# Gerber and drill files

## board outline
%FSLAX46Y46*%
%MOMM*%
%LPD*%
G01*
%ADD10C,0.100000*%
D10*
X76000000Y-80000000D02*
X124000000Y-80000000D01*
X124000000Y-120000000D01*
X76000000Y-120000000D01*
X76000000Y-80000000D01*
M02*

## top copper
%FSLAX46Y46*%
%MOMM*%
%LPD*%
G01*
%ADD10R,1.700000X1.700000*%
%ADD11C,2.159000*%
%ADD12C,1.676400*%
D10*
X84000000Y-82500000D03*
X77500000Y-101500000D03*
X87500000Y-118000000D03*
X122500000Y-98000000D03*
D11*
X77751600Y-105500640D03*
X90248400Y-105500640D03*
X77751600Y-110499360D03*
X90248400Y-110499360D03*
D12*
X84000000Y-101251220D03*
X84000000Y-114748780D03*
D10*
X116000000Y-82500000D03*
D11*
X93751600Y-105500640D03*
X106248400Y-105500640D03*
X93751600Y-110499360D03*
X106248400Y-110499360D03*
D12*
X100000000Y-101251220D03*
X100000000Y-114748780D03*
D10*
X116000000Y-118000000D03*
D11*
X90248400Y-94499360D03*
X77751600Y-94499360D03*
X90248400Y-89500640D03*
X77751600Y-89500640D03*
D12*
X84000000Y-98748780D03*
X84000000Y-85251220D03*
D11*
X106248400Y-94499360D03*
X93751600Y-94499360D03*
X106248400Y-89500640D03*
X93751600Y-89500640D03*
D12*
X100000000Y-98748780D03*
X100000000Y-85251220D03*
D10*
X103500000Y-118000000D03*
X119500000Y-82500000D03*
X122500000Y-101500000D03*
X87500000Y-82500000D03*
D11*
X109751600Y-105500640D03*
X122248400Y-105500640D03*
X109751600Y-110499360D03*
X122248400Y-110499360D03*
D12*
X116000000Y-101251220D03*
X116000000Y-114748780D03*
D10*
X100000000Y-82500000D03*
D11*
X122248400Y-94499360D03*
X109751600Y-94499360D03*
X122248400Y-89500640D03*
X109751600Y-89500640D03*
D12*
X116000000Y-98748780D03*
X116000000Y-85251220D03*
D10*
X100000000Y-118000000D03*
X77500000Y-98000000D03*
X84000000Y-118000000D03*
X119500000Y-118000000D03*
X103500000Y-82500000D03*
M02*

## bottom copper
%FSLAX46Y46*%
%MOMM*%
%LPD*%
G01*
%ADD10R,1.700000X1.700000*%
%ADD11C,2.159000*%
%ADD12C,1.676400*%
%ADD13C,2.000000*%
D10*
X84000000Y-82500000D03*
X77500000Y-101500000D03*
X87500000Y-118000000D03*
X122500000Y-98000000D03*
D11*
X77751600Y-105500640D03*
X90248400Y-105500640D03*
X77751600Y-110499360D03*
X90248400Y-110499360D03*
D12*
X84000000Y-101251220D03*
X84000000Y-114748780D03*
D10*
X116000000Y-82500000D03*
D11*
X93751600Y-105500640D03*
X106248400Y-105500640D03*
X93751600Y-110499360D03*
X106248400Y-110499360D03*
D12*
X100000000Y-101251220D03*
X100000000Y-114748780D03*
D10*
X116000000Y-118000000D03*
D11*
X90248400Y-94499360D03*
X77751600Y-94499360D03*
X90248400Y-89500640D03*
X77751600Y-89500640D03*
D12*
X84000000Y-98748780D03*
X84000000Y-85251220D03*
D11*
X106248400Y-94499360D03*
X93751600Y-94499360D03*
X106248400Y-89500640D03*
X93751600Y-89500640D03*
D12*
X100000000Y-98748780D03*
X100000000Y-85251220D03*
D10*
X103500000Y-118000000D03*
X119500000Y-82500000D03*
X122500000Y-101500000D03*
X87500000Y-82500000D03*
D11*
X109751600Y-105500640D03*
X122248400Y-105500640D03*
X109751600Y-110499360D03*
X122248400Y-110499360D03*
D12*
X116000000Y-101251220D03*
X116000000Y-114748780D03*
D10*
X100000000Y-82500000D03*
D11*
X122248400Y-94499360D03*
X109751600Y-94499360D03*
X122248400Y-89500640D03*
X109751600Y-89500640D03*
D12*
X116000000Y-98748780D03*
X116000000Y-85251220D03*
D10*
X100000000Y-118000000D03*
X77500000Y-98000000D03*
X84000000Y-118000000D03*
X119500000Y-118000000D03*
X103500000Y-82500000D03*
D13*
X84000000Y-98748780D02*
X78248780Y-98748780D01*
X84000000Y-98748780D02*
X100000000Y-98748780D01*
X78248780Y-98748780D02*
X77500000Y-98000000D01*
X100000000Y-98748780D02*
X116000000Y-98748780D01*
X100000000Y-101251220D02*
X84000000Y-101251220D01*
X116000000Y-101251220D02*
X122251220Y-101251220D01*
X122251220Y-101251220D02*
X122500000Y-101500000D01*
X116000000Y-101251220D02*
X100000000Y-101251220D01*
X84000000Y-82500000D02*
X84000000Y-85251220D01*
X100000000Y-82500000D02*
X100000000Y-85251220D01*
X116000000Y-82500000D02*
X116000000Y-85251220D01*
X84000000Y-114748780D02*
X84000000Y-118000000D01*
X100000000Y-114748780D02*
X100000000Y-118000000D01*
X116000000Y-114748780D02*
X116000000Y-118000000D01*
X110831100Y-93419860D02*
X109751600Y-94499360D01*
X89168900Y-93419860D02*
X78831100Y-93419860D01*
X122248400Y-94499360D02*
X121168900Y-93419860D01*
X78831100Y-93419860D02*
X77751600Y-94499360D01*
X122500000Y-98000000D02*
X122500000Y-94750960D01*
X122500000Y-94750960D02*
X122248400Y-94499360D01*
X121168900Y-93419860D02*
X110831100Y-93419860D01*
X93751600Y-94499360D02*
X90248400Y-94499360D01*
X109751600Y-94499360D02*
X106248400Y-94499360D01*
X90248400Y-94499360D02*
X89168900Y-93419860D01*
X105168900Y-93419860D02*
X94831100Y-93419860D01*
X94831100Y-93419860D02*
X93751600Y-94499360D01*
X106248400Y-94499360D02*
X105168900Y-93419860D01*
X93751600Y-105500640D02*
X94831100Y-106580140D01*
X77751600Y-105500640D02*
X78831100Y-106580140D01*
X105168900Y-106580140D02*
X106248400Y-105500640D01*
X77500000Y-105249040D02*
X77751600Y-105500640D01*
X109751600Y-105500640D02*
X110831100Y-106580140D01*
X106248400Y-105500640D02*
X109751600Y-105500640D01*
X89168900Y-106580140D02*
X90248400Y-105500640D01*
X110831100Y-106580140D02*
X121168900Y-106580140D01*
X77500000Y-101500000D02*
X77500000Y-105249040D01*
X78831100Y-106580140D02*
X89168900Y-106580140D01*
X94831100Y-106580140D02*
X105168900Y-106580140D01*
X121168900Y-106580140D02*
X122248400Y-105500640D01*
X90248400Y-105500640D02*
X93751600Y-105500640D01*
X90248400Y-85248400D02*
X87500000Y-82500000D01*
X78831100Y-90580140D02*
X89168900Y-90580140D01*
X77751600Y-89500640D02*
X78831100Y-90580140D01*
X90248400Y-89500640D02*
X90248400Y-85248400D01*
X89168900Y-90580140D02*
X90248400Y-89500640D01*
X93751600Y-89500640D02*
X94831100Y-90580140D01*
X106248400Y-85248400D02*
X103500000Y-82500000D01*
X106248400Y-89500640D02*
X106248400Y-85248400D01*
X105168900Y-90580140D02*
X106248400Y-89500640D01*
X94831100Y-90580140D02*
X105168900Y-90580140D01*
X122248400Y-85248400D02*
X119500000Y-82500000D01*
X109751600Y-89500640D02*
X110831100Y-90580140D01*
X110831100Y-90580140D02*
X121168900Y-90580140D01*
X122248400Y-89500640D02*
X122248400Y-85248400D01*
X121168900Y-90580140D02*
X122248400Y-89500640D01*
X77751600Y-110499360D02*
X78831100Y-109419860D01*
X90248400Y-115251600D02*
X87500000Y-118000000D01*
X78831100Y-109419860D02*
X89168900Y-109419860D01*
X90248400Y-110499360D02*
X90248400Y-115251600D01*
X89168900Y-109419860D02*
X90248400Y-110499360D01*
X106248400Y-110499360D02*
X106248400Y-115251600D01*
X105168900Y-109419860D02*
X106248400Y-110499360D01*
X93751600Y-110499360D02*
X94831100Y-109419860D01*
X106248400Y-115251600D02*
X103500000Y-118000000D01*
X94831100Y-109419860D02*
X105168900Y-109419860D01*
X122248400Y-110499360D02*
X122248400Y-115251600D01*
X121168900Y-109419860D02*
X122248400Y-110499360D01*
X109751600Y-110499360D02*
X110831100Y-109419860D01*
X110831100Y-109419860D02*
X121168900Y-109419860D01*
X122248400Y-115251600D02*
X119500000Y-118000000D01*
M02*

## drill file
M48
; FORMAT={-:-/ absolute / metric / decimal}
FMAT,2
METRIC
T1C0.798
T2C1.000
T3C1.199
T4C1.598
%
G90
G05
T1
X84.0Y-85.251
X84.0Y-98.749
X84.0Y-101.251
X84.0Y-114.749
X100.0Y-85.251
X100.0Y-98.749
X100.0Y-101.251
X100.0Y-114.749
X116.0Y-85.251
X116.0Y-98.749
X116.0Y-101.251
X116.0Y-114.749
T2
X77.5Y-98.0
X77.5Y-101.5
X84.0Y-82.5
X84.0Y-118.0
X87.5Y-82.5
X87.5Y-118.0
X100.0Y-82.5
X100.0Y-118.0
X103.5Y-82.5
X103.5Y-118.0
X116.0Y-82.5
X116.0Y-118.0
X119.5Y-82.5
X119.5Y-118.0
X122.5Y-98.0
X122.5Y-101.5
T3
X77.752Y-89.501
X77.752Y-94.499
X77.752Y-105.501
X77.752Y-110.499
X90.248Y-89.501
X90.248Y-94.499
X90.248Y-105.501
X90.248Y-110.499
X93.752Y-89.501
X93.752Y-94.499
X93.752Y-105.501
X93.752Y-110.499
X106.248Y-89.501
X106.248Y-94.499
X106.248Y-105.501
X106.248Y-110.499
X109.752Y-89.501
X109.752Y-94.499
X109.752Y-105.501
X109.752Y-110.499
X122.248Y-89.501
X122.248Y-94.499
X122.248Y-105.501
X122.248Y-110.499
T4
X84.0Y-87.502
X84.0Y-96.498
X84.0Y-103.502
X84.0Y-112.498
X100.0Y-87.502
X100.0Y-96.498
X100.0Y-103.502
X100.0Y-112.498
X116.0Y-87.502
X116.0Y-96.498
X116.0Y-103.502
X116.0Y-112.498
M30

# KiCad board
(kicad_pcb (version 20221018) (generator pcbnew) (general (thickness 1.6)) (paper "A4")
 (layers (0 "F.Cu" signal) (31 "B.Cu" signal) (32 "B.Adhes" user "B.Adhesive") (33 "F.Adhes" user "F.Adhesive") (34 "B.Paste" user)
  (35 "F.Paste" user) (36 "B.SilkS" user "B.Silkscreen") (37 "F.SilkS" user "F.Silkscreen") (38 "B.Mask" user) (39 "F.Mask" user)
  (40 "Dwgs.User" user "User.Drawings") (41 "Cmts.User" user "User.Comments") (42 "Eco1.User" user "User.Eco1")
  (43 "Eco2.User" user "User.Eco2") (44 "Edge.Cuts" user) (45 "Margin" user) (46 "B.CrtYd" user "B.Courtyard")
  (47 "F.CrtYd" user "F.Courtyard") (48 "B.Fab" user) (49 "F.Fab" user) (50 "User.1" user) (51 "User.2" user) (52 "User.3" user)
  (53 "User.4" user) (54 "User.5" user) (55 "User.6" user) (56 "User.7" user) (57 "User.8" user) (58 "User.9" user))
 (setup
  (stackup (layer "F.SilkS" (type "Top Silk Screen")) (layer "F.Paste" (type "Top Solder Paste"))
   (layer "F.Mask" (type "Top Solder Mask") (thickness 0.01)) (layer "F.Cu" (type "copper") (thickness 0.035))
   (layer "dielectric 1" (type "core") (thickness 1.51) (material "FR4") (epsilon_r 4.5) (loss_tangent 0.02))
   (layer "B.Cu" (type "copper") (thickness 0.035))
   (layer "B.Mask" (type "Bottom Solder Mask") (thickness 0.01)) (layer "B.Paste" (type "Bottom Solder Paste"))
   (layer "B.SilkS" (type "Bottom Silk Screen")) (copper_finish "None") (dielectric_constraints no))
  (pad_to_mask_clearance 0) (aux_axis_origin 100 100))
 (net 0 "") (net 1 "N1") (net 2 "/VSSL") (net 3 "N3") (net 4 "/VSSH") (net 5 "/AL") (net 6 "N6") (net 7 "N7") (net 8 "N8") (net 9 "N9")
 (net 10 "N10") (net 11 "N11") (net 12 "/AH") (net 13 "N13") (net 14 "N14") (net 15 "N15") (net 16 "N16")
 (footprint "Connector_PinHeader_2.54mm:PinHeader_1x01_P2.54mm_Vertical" (layer "F.Cu") (at 84 82.5)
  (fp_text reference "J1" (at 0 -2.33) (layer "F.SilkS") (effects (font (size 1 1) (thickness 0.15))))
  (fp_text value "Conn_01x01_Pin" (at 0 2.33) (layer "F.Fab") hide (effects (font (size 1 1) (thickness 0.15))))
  (pad "1" thru_hole rect (at 0 0) (size 1.7 1.7) (drill 1) (layers "*.Cu" "*.Mask") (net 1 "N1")))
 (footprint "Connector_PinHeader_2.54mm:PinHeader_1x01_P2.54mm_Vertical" (layer "F.Cu") (at 77.5 101.5)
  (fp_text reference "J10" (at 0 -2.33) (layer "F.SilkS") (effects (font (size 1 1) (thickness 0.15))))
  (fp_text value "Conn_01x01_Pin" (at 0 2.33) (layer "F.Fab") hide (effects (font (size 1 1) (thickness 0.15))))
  (pad "1" thru_hole rect (at 0 0) (size 1.7 1.7) (drill 1) (layers "*.Cu" "*.Mask") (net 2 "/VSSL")))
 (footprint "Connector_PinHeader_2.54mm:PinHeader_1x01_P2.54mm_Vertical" (layer "F.Cu") (at 87.5 118)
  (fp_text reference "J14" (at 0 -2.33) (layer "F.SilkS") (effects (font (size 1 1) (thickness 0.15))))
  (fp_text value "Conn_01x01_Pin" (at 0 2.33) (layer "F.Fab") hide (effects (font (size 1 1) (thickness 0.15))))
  (pad "1" thru_hole rect (at 0 0) (size 1.7 1.7) (drill 1) (layers "*.Cu" "*.Mask") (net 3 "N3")))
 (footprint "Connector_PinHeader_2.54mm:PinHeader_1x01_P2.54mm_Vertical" (layer "F.Cu") (at 122.5 98)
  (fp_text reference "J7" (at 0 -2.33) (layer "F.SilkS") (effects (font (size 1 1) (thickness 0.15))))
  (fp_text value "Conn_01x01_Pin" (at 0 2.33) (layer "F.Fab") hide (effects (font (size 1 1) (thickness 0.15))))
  (pad "1" thru_hole rect (at 0 0) (size 1.7 1.7) (drill 1) (layers "*.Cu" "*.Mask") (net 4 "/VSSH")))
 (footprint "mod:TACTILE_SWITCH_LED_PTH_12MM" (layer "F.Cu") (at 84 108)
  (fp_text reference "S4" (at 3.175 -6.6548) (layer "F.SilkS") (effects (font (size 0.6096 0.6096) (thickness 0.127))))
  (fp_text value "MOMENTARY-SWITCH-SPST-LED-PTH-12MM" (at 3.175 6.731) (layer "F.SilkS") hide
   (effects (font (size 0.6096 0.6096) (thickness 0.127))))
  (pad "" np_thru_hole circle (at 0 -4.49834) (size 1.59766 1.59766) (drill 1.59766) (layers "*.Cu" "*.Mask") (solder_mask_margin 0.1016))
  (pad "" np_thru_hole circle (at 0 4.49834) (size 1.59766 1.59766) (drill 1.59766) (layers "*.Cu" "*.Mask") (solder_mask_margin 0.1016))
  (pad "1" thru_hole circle (at -6.2484 -2.49936) (size 2.159 2.159) (drill 1.19888) (layers "*.Cu" "*.Mask") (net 2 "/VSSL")
   (solder_mask_margin 0.1016))
  (pad "2" thru_hole circle (at 6.2484 -2.49936) (size 2.159 2.159) (drill 1.19888) (layers "*.Cu" "*.Mask") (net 2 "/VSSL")
   (solder_mask_margin 0.1016))
  (pad "3" thru_hole circle (at -6.2484 2.49936) (size 2.159 2.159) (drill 1.19888) (layers "*.Cu" "*.Mask") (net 3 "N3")
   (solder_mask_margin 0.1016))
  (pad "4" thru_hole circle (at 6.2484 2.49936) (size 2.159 2.159) (drill 1.19888) (layers "*.Cu" "*.Mask") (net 3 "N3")
   (solder_mask_margin 0.1016))
  (pad "A" thru_hole circle (at 0 -6.74878) (size 1.6764 1.6764) (drill 0.79756) (layers "*.Cu" "*.Mask") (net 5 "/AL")
   (solder_mask_margin 0.1016))
  (pad "C" thru_hole circle (at 0 6.74878) (size 1.6764 1.6764) (drill 0.79756) (layers "*.Cu" "*.Mask") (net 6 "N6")
   (solder_mask_margin 0.1016)))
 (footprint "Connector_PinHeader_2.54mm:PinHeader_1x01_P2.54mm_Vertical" (layer "F.Cu") (at 116 82.5)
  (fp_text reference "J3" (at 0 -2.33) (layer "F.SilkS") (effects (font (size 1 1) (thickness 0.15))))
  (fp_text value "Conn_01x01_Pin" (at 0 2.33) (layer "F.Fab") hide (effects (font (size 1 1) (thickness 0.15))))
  (pad "1" thru_hole rect (at 0 0) (size 1.7 1.7) (drill 1) (layers "*.Cu" "*.Mask") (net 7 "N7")))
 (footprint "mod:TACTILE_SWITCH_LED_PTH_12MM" (layer "F.Cu") (at 100 108)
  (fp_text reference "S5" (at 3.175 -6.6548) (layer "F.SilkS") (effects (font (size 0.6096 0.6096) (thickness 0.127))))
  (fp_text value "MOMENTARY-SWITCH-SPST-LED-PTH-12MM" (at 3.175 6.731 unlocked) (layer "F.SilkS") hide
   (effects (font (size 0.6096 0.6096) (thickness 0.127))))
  (pad "" np_thru_hole circle (at 0 -4.49834) (size 1.59766 1.59766) (drill 1.59766) (layers "*.Cu" "*.Mask") (solder_mask_margin 0.1016))
  (pad "" np_thru_hole circle (at 0 4.49834) (size 1.59766 1.59766) (drill 1.59766) (layers "*.Cu" "*.Mask") (solder_mask_margin 0.1016))
  (pad "1" thru_hole circle (at -6.2484 -2.49936) (size 2.159 2.159) (drill 1.19888) (layers "*.Cu" "*.Mask") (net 2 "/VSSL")
   (solder_mask_margin 0.1016))
  (pad "2" thru_hole circle (at 6.2484 -2.49936) (size 2.159 2.159) (drill 1.19888) (layers "*.Cu" "*.Mask") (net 2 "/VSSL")
   (solder_mask_margin 0.1016))
  (pad "3" thru_hole circle (at -6.2484 2.49936) (size 2.159 2.159) (drill 1.19888) (layers "*.Cu" "*.Mask") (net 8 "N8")
   (solder_mask_margin 0.1016))
  (pad "4" thru_hole circle (at 6.2484 2.49936) (size 2.159 2.159) (drill 1.19888) (layers "*.Cu" "*.Mask") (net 8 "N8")
   (solder_mask_margin 0.1016))
  (pad "A" thru_hole circle (at 0 -6.74878) (size 1.6764 1.6764) (drill 0.79756) (layers "*.Cu" "*.Mask") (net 5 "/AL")
   (solder_mask_margin 0.1016))
  (pad "C" thru_hole circle (at 0 6.74878) (size 1.6764 1.6764) (drill 0.79756) (layers "*.Cu" "*.Mask") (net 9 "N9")
   (solder_mask_margin 0.1016)))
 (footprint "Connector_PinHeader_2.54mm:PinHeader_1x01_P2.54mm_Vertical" (layer "F.Cu") (at 116 118)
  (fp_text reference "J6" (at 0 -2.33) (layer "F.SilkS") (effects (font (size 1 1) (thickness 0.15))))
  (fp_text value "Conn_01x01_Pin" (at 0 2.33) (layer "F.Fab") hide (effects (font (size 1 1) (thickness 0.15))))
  (pad "1" thru_hole rect (at 0 0) (size 1.7 1.7) (drill 1) (layers "*.Cu" "*.Mask") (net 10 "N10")))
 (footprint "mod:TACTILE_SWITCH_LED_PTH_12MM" (layer "F.Cu") (at 84 92 180)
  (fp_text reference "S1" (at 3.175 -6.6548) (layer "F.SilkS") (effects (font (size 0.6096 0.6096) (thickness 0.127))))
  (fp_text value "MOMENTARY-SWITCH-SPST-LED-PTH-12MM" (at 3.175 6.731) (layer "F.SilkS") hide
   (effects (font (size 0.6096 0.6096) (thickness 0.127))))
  (pad "" np_thru_hole circle (at 0 -4.49834 180) (size 1.59766 1.59766) (drill 1.59766) (layers "*.Cu" "*.Mask")
   (solder_mask_margin 0.1016))
  (pad "" np_thru_hole circle (at 0 4.49834 180) (size 1.59766 1.59766) (drill 1.59766) (layers "*.Cu" "*.Mask") (solder_mask_margin 0.1016))
  (pad "1" thru_hole circle (at -6.2484 -2.49936 180) (size 2.159 2.159) (drill 1.19888) (layers "*.Cu" "*.Mask") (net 4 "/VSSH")
   (solder_mask_margin 0.1016))
  (pad "2" thru_hole circle (at 6.2484 -2.49936 180) (size 2.159 2.159) (drill 1.19888) (layers "*.Cu" "*.Mask") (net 4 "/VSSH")
   (solder_mask_margin 0.1016))
  (pad "3" thru_hole circle (at -6.2484 2.49936 180) (size 2.159 2.159) (drill 1.19888) (layers "*.Cu" "*.Mask") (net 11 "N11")
   (solder_mask_margin 0.1016))
  (pad "4" thru_hole circle (at 6.2484 2.49936 180) (size 2.159 2.159) (drill 1.19888) (layers "*.Cu" "*.Mask") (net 11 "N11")
   (solder_mask_margin 0.1016))
  (pad "A" thru_hole circle (at 0 -6.74878 180) (size 1.6764 1.6764) (drill 0.79756) (layers "*.Cu" "*.Mask") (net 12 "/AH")
   (solder_mask_margin 0.1016))
  (pad "C" thru_hole circle (at 0 6.74878 180) (size 1.6764 1.6764) (drill 0.79756) (layers "*.Cu" "*.Mask") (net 1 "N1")
   (solder_mask_margin 0.1016)))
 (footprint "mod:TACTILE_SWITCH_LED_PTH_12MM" (layer "F.Cu") (at 100 92 180)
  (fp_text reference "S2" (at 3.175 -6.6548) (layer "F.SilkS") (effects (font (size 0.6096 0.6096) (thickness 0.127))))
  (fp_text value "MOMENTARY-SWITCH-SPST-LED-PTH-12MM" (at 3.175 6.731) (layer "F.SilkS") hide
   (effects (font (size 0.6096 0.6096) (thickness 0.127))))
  (pad "" np_thru_hole circle (at 0 -4.49834 180) (size 1.59766 1.59766) (drill 1.59766) (layers "*.Cu" "*.Mask")
   (solder_mask_margin 0.1016))
  (pad "" np_thru_hole circle (at 0 4.49834 180) (size 1.59766 1.59766) (drill 1.59766) (layers "*.Cu" "*.Mask") (solder_mask_margin 0.1016))
  (pad "1" thru_hole circle (at -6.2484 -2.49936 180) (size 2.159 2.159) (drill 1.19888) (layers "*.Cu" "*.Mask") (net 4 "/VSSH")
   (solder_mask_margin 0.1016))
  (pad "2" thru_hole circle (at 6.2484 -2.49936 180) (size 2.159 2.159) (drill 1.19888) (layers "*.Cu" "*.Mask") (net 4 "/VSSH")
   (solder_mask_margin 0.1016))
  (pad "3" thru_hole circle (at -6.2484 2.49936 180) (size 2.159 2.159) (drill 1.19888) (layers "*.Cu" "*.Mask") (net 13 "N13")
   (solder_mask_margin 0.1016))
  (pad "4" thru_hole circle (at 6.2484 2.49936 180) (size 2.159 2.159) (drill 1.19888) (layers "*.Cu" "*.Mask") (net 13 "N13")
   (solder_mask_margin 0.1016))
  (pad "A" thru_hole circle (at 0 -6.74878 180) (size 1.6764 1.6764) (drill 0.79756) (layers "*.Cu" "*.Mask") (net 12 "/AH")
   (solder_mask_margin 0.1016))
  (pad "C" thru_hole circle (at 0 6.74878 180) (size 1.6764 1.6764) (drill 0.79756) (layers "*.Cu" "*.Mask") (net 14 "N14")
   (solder_mask_margin 0.1016)))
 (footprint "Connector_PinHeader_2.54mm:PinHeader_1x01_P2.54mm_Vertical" (layer "F.Cu") (at 103.5 118)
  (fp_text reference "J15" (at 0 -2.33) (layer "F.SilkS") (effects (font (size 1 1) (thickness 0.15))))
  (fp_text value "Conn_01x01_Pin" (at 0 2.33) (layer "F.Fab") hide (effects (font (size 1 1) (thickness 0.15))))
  (pad "1" thru_hole rect (at 0 0) (size 1.7 1.7) (drill 1) (layers "*.Cu" "*.Mask") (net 8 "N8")))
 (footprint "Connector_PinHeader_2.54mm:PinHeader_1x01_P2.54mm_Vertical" (layer "F.Cu") (at 119.5 82.5)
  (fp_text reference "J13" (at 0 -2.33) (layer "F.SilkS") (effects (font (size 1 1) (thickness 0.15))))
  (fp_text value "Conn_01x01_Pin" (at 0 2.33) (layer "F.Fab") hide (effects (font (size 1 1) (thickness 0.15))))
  (pad "1" thru_hole rect (at 0 0) (size 1.7 1.7) (drill 1) (layers "*.Cu" "*.Mask") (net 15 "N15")))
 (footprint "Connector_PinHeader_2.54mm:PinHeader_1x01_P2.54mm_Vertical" (layer "F.Cu") (at 122.5 101.5)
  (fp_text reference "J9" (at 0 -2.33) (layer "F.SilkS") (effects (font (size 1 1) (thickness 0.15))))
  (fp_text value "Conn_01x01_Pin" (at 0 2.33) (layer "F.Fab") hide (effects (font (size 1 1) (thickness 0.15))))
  (pad "1" thru_hole rect (at 0 0) (size 1.7 1.7) (drill 1) (layers "*.Cu" "*.Mask") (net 5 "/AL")))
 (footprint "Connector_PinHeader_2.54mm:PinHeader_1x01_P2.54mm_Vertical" (layer "F.Cu") (at 87.5 82.5)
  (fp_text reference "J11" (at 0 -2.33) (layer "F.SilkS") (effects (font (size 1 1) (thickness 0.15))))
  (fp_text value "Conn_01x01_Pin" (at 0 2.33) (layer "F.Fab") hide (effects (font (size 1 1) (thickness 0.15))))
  (pad "1" thru_hole rect (at 0 0) (size 1.7 1.7) (drill 1) (layers "*.Cu" "*.Mask") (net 11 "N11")))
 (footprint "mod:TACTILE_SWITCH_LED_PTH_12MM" (layer "F.Cu") (at 116 108)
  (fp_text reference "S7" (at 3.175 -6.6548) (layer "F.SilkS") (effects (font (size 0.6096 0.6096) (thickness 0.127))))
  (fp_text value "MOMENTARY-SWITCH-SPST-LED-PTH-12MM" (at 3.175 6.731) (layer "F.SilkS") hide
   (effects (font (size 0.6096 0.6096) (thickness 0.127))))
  (pad "" np_thru_hole circle (at 0 -4.49834) (size 1.59766 1.59766) (drill 1.59766) (layers "*.Cu" "*.Mask") (solder_mask_margin 0.1016))
  (pad "" np_thru_hole circle (at 0 4.49834) (size 1.59766 1.59766) (drill 1.59766) (layers "*.Cu" "*.Mask") (solder_mask_margin 0.1016))
  (pad "1" thru_hole circle (at -6.2484 -2.49936) (size 2.159 2.159) (drill 1.19888) (layers "*.Cu" "*.Mask") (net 2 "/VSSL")
   (solder_mask_margin 0.1016))
  (pad "2" thru_hole circle (at 6.2484 -2.49936) (size 2.159 2.159) (drill 1.19888) (layers "*.Cu" "*.Mask") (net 2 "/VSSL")
   (solder_mask_margin 0.1016))
  (pad "3" thru_hole circle (at -6.2484 2.49936) (size 2.159 2.159) (drill 1.19888) (layers "*.Cu" "*.Mask") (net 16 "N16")
   (solder_mask_margin 0.1016))
  (pad "4" thru_hole circle (at 6.2484 2.49936) (size 2.159 2.159) (drill 1.19888) (layers "*.Cu" "*.Mask") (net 16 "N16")
   (solder_mask_margin 0.1016))
  (pad "A" thru_hole circle (at 0 -6.74878) (size 1.6764 1.6764) (drill 0.79756) (layers "*.Cu" "*.Mask") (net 5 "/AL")
   (solder_mask_margin 0.1016))
  (pad "C" thru_hole circle (at 0 6.74878) (size 1.6764 1.6764) (drill 0.79756) (layers "*.Cu" "*.Mask") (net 10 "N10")
   (solder_mask_margin 0.1016)))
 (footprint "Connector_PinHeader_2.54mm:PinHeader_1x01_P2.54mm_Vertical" (layer "F.Cu") (at 100 82.5)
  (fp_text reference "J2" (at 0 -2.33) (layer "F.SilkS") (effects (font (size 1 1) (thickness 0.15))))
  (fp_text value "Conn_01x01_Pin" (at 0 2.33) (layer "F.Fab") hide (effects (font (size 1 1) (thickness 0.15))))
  (pad "1" thru_hole rect (at 0 0) (size 1.7 1.7) (drill 1) (layers "*.Cu" "*.Mask") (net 14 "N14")))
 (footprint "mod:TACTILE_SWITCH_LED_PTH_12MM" (layer "F.Cu") (at 116 92 180)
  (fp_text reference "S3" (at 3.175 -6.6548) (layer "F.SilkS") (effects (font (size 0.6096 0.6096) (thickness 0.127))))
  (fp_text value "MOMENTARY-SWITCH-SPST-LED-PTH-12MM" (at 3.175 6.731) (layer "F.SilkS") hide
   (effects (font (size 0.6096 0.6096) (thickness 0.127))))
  (pad "" np_thru_hole circle (at 0 -4.49834 180) (size 1.59766 1.59766) (drill 1.59766) (layers "*.Cu" "*.Mask")
   (solder_mask_margin 0.1016))
  (pad "" np_thru_hole circle (at 0 4.49834 180) (size 1.59766 1.59766) (drill 1.59766) (layers "*.Cu" "*.Mask") (solder_mask_margin 0.1016))
  (pad "1" thru_hole circle (at -6.2484 -2.49936 180) (size 2.159 2.159) (drill 1.19888) (layers "*.Cu" "*.Mask") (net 4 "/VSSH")
   (solder_mask_margin 0.1016))
  (pad "2" thru_hole circle (at 6.2484 -2.49936 180) (size 2.159 2.159) (drill 1.19888) (layers "*.Cu" "*.Mask") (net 4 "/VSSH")
   (solder_mask_margin 0.1016))
  (pad "3" thru_hole circle (at -6.2484 2.49936 180) (size 2.159 2.159) (drill 1.19888) (layers "*.Cu" "*.Mask") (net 15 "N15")
   (solder_mask_margin 0.1016))
  (pad "4" thru_hole circle (at 6.2484 2.49936 180) (size 2.159 2.159) (drill 1.19888) (layers "*.Cu" "*.Mask") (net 15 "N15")
   (solder_mask_margin 0.1016))
  (pad "A" thru_hole circle (at 0 -6.74878 180) (size 1.6764 1.6764) (drill 0.79756) (layers "*.Cu" "*.Mask") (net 12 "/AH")
   (solder_mask_margin 0.1016))
  (pad "C" thru_hole circle (at 0 6.74878 180) (size 1.6764 1.6764) (drill 0.79756) (layers "*.Cu" "*.Mask") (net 7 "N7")
   (solder_mask_margin 0.1016)))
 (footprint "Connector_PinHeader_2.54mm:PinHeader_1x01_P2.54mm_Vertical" (layer "F.Cu") (at 100 118)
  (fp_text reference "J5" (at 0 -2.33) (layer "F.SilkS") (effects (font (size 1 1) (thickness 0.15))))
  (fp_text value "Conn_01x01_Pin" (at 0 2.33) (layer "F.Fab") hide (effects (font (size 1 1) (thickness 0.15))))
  (pad "1" thru_hole rect (at 0 0) (size 1.7 1.7) (drill 1) (layers "*.Cu" "*.Mask") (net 9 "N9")))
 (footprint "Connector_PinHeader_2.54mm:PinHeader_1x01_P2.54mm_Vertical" (layer "F.Cu") (at 77.5 98)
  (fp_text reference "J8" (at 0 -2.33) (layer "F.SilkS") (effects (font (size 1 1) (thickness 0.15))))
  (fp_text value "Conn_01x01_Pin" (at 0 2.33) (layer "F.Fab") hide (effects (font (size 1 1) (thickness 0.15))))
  (pad "1" thru_hole rect (at 0 0) (size 1.7 1.7) (drill 1) (layers "*.Cu" "*.Mask") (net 12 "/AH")))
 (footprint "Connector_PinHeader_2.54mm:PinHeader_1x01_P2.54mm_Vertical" (layer "F.Cu") (at 84 118)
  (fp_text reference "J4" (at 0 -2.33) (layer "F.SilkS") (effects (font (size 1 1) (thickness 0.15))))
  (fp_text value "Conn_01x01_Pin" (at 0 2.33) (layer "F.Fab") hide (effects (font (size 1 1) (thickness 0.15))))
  (pad "1" thru_hole rect (at 0 0) (size 1.7 1.7) (drill 1) (layers "*.Cu" "*.Mask") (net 6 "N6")))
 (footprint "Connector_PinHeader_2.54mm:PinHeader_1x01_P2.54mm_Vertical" (layer "F.Cu") (at 119.5 118)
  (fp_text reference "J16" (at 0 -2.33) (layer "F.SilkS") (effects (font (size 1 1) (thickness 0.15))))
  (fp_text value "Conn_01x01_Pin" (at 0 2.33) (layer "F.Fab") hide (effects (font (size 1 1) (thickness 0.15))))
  (pad "1" thru_hole rect (at 0 0) (size 1.7 1.7) (drill 1) (layers "*.Cu" "*.Mask") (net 16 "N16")))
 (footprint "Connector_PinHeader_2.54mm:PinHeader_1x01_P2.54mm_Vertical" (layer "F.Cu") (at 103.5 82.5)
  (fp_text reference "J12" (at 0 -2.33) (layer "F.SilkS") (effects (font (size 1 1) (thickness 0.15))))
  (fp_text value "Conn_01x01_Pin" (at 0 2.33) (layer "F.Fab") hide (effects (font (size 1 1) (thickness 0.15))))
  (pad "1" thru_hole rect (at 0 0) (size 1.7 1.7) (drill 1) (layers "*.Cu" "*.Mask") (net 13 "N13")))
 (gr_rect (start 76 80) (end 124 120) (stroke (width 0.1) (type default)) (fill none) (layer "Edge.Cuts"))
 (segment (start 84 98.74878) (end 78.24878 98.74878) (width 2) (layer "B.Cu") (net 12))
 (segment (start 84 98.74878) (end 100 98.74878) (width 2) (layer "B.Cu") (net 12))
 (segment (start 78.24878 98.74878) (end 77.5 98) (width 2) (layer "B.Cu") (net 12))
 (segment (start 100 98.74878) (end 116 98.74878) (width 2) (layer "B.Cu") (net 12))
 (segment (start 100 101.25122) (end 84 101.25122) (width 2) (layer "B.Cu") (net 5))
 (segment (start 116 101.25122) (end 122.25122 101.25122) (width 2) (layer "B.Cu") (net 5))
 (segment (start 122.25122 101.25122) (end 122.5 101.5) (width 2) (layer "B.Cu") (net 5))
 (segment (start 116 101.25122) (end 100 101.25122) (width 2) (layer "B.Cu") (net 5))
 (segment (start 84 82.5) (end 84 85.25122) (width 2) (layer "B.Cu") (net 1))
 (segment (start 100 82.5) (end 100 85.25122) (width 2) (layer "B.Cu") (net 14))
 (segment (start 116 82.5) (end 116 85.25122) (width 2) (layer "B.Cu") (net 7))
 (segment (start 84 114.74878) (end 84 118) (width 2) (layer "B.Cu") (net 6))
 (segment (start 100 114.74878) (end 100 118) (width 2) (layer "B.Cu") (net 9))
 (segment (start 116 114.74878) (end 116 118) (width 2) (layer "B.Cu") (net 10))
 (segment (start 110.8311 93.41986) (end 109.7516 94.49936) (width 2) (layer "B.Cu") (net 4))
 (segment (start 89.1689 93.41986) (end 78.8311 93.41986) (width 2) (layer "B.Cu") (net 4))
 (segment (start 122.2484 94.49936) (end 121.1689 93.41986) (width 2) (layer "B.Cu") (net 4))
 (segment (start 78.8311 93.41986) (end 77.7516 94.49936) (width 2) (layer "B.Cu") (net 4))
 (segment (start 122.5 98) (end 122.5 94.75096) (width 2) (layer "B.Cu") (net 4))
 (segment (start 122.5 94.75096) (end 122.2484 94.49936) (width 2) (layer "B.Cu") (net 4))
 (segment (start 121.1689 93.41986) (end 110.8311 93.41986) (width 2) (layer "B.Cu") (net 4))
 (segment (start 93.7516 94.49936) (end 90.2484 94.49936) (width 2) (layer "B.Cu") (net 4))
 (segment (start 109.7516 94.49936) (end 106.2484 94.49936) (width 2) (layer "B.Cu") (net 4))
 (segment (start 90.2484 94.49936) (end 89.1689 93.41986) (width 2) (layer "B.Cu") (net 4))
 (segment (start 105.1689 93.41986) (end 94.8311 93.41986) (width 2) (layer "B.Cu") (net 4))
 (segment (start 94.8311 93.41986) (end 93.7516 94.49936) (width 2) (layer "B.Cu") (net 4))
 (segment (start 106.2484 94.49936) (end 105.1689 93.41986) (width 2) (layer "B.Cu") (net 4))
 (segment (start 93.7516 105.50064) (end 94.8311 106.58014) (width 2) (layer "B.Cu") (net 2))
 (segment (start 77.7516 105.50064) (end 78.8311 106.58014) (width 2) (layer "B.Cu") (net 2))
 (segment (start 105.1689 106.58014) (end 106.2484 105.50064) (width 2) (layer "B.Cu") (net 2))
 (segment (start 77.5 105.24904) (end 77.7516 105.50064) (width 2) (layer "B.Cu") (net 2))
 (segment (start 109.7516 105.50064) (end 110.8311 106.58014) (width 2) (layer "B.Cu") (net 2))
 (segment (start 106.2484 105.50064) (end 109.7516 105.50064) (width 2) (layer "B.Cu") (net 2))
 (segment (start 89.1689 106.58014) (end 90.2484 105.50064) (width 2) (layer "B.Cu") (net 2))
 (segment (start 110.8311 106.58014) (end 121.1689 106.58014) (width 2) (layer "B.Cu") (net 2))
 (segment (start 77.5 101.5) (end 77.5 105.24904) (width 2) (layer "B.Cu") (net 2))
 (segment (start 78.8311 106.58014) (end 89.1689 106.58014) (width 2) (layer "B.Cu") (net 2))
 (segment (start 94.8311 106.58014) (end 105.1689 106.58014) (width 2) (layer "B.Cu") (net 2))
 (segment (start 121.1689 106.58014) (end 122.2484 105.50064) (width 2) (layer "B.Cu") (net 2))
 (segment (start 90.2484 105.50064) (end 93.7516 105.50064) (width 2) (layer "B.Cu") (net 2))
 (segment (start 90.2484 85.2484) (end 87.5 82.5) (width 2) (layer "B.Cu") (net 11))
 (segment (start 78.8311 90.58014) (end 89.1689 90.58014) (width 2) (layer "B.Cu") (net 11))
 (segment (start 77.7516 89.50064) (end 78.8311 90.58014) (width 2) (layer "B.Cu") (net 11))
 (segment (start 90.2484 89.50064) (end 90.2484 85.2484) (width 2) (layer "B.Cu") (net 11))
 (segment (start 89.1689 90.58014) (end 90.2484 89.50064) (width 2) (layer "B.Cu") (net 11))
 (segment (start 93.7516 89.50064) (end 94.8311 90.58014) (width 2) (layer "B.Cu") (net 13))
 (segment (start 106.2484 85.2484) (end 103.5 82.5) (width 2) (layer "B.Cu") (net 13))
 (segment (start 106.2484 89.50064) (end 106.2484 85.2484) (width 2) (layer "B.Cu") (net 13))
 (segment (start 105.1689 90.58014) (end 106.2484 89.50064) (width 2) (layer "B.Cu") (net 13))
 (segment (start 94.8311 90.58014) (end 105.1689 90.58014) (width 2) (layer "B.Cu") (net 13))
 (segment (start 122.2484 85.2484) (end 119.5 82.5) (width 2) (layer "B.Cu") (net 15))
 (segment (start 109.7516 89.50064) (end 110.8311 90.58014) (width 2) (layer "B.Cu") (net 15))
 (segment (start 110.8311 90.58014) (end 121.1689 90.58014) (width 2) (layer "B.Cu") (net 15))
 (segment (start 122.2484 89.50064) (end 122.2484 85.2484) (width 2) (layer "B.Cu") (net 15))
 (segment (start 121.1689 90.58014) (end 122.2484 89.50064) (width 2) (layer "B.Cu") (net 15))
 (segment (start 77.7516 110.49936) (end 78.8311 109.41986) (width 2) (layer "B.Cu") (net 3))
 (segment (start 90.2484 115.2516) (end 87.5 118) (width 2) (layer "B.Cu") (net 3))
 (segment (start 78.8311 109.41986) (end 89.1689 109.41986) (width 2) (layer "B.Cu") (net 3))
 (segment (start 90.2484 110.49936) (end 90.2484 115.2516) (width 2) (layer "B.Cu") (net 3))
 (segment (start 89.1689 109.41986) (end 90.2484 110.49936) (width 2) (layer "B.Cu") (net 3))
 (segment (start 106.2484 110.49936) (end 106.2484 115.2516) (width 2) (layer "B.Cu") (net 8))
 (segment (start 105.1689 109.41986) (end 106.2484 110.49936) (width 2) (layer "B.Cu") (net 8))
 (segment (start 93.7516 110.49936) (end 94.8311 109.41986) (width 2) (layer "B.Cu") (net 8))
 (segment (start 106.2484 115.2516) (end 103.5 118) (width 2) (layer "B.Cu") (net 8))
 (segment (start 94.8311 109.41986) (end 105.1689 109.41986) (width 2) (layer "B.Cu") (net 8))
 (segment (start 122.2484 110.49936) (end 122.2484 115.2516) (width 2) (layer "B.Cu") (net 16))
 (segment (start 121.1689 109.41986) (end 122.2484 110.49936) (width 2) (layer "B.Cu") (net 16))
 (segment (start 109.7516 110.49936) (end 110.8311 109.41986) (width 2) (layer "B.Cu") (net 16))
 (segment (start 110.8311 109.41986) (end 121.1689 109.41986) (width 2) (layer "B.Cu") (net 16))
 (segment (start 122.2484 115.2516) (end 119.5 118) (width 2) (layer "B.Cu") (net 16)))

